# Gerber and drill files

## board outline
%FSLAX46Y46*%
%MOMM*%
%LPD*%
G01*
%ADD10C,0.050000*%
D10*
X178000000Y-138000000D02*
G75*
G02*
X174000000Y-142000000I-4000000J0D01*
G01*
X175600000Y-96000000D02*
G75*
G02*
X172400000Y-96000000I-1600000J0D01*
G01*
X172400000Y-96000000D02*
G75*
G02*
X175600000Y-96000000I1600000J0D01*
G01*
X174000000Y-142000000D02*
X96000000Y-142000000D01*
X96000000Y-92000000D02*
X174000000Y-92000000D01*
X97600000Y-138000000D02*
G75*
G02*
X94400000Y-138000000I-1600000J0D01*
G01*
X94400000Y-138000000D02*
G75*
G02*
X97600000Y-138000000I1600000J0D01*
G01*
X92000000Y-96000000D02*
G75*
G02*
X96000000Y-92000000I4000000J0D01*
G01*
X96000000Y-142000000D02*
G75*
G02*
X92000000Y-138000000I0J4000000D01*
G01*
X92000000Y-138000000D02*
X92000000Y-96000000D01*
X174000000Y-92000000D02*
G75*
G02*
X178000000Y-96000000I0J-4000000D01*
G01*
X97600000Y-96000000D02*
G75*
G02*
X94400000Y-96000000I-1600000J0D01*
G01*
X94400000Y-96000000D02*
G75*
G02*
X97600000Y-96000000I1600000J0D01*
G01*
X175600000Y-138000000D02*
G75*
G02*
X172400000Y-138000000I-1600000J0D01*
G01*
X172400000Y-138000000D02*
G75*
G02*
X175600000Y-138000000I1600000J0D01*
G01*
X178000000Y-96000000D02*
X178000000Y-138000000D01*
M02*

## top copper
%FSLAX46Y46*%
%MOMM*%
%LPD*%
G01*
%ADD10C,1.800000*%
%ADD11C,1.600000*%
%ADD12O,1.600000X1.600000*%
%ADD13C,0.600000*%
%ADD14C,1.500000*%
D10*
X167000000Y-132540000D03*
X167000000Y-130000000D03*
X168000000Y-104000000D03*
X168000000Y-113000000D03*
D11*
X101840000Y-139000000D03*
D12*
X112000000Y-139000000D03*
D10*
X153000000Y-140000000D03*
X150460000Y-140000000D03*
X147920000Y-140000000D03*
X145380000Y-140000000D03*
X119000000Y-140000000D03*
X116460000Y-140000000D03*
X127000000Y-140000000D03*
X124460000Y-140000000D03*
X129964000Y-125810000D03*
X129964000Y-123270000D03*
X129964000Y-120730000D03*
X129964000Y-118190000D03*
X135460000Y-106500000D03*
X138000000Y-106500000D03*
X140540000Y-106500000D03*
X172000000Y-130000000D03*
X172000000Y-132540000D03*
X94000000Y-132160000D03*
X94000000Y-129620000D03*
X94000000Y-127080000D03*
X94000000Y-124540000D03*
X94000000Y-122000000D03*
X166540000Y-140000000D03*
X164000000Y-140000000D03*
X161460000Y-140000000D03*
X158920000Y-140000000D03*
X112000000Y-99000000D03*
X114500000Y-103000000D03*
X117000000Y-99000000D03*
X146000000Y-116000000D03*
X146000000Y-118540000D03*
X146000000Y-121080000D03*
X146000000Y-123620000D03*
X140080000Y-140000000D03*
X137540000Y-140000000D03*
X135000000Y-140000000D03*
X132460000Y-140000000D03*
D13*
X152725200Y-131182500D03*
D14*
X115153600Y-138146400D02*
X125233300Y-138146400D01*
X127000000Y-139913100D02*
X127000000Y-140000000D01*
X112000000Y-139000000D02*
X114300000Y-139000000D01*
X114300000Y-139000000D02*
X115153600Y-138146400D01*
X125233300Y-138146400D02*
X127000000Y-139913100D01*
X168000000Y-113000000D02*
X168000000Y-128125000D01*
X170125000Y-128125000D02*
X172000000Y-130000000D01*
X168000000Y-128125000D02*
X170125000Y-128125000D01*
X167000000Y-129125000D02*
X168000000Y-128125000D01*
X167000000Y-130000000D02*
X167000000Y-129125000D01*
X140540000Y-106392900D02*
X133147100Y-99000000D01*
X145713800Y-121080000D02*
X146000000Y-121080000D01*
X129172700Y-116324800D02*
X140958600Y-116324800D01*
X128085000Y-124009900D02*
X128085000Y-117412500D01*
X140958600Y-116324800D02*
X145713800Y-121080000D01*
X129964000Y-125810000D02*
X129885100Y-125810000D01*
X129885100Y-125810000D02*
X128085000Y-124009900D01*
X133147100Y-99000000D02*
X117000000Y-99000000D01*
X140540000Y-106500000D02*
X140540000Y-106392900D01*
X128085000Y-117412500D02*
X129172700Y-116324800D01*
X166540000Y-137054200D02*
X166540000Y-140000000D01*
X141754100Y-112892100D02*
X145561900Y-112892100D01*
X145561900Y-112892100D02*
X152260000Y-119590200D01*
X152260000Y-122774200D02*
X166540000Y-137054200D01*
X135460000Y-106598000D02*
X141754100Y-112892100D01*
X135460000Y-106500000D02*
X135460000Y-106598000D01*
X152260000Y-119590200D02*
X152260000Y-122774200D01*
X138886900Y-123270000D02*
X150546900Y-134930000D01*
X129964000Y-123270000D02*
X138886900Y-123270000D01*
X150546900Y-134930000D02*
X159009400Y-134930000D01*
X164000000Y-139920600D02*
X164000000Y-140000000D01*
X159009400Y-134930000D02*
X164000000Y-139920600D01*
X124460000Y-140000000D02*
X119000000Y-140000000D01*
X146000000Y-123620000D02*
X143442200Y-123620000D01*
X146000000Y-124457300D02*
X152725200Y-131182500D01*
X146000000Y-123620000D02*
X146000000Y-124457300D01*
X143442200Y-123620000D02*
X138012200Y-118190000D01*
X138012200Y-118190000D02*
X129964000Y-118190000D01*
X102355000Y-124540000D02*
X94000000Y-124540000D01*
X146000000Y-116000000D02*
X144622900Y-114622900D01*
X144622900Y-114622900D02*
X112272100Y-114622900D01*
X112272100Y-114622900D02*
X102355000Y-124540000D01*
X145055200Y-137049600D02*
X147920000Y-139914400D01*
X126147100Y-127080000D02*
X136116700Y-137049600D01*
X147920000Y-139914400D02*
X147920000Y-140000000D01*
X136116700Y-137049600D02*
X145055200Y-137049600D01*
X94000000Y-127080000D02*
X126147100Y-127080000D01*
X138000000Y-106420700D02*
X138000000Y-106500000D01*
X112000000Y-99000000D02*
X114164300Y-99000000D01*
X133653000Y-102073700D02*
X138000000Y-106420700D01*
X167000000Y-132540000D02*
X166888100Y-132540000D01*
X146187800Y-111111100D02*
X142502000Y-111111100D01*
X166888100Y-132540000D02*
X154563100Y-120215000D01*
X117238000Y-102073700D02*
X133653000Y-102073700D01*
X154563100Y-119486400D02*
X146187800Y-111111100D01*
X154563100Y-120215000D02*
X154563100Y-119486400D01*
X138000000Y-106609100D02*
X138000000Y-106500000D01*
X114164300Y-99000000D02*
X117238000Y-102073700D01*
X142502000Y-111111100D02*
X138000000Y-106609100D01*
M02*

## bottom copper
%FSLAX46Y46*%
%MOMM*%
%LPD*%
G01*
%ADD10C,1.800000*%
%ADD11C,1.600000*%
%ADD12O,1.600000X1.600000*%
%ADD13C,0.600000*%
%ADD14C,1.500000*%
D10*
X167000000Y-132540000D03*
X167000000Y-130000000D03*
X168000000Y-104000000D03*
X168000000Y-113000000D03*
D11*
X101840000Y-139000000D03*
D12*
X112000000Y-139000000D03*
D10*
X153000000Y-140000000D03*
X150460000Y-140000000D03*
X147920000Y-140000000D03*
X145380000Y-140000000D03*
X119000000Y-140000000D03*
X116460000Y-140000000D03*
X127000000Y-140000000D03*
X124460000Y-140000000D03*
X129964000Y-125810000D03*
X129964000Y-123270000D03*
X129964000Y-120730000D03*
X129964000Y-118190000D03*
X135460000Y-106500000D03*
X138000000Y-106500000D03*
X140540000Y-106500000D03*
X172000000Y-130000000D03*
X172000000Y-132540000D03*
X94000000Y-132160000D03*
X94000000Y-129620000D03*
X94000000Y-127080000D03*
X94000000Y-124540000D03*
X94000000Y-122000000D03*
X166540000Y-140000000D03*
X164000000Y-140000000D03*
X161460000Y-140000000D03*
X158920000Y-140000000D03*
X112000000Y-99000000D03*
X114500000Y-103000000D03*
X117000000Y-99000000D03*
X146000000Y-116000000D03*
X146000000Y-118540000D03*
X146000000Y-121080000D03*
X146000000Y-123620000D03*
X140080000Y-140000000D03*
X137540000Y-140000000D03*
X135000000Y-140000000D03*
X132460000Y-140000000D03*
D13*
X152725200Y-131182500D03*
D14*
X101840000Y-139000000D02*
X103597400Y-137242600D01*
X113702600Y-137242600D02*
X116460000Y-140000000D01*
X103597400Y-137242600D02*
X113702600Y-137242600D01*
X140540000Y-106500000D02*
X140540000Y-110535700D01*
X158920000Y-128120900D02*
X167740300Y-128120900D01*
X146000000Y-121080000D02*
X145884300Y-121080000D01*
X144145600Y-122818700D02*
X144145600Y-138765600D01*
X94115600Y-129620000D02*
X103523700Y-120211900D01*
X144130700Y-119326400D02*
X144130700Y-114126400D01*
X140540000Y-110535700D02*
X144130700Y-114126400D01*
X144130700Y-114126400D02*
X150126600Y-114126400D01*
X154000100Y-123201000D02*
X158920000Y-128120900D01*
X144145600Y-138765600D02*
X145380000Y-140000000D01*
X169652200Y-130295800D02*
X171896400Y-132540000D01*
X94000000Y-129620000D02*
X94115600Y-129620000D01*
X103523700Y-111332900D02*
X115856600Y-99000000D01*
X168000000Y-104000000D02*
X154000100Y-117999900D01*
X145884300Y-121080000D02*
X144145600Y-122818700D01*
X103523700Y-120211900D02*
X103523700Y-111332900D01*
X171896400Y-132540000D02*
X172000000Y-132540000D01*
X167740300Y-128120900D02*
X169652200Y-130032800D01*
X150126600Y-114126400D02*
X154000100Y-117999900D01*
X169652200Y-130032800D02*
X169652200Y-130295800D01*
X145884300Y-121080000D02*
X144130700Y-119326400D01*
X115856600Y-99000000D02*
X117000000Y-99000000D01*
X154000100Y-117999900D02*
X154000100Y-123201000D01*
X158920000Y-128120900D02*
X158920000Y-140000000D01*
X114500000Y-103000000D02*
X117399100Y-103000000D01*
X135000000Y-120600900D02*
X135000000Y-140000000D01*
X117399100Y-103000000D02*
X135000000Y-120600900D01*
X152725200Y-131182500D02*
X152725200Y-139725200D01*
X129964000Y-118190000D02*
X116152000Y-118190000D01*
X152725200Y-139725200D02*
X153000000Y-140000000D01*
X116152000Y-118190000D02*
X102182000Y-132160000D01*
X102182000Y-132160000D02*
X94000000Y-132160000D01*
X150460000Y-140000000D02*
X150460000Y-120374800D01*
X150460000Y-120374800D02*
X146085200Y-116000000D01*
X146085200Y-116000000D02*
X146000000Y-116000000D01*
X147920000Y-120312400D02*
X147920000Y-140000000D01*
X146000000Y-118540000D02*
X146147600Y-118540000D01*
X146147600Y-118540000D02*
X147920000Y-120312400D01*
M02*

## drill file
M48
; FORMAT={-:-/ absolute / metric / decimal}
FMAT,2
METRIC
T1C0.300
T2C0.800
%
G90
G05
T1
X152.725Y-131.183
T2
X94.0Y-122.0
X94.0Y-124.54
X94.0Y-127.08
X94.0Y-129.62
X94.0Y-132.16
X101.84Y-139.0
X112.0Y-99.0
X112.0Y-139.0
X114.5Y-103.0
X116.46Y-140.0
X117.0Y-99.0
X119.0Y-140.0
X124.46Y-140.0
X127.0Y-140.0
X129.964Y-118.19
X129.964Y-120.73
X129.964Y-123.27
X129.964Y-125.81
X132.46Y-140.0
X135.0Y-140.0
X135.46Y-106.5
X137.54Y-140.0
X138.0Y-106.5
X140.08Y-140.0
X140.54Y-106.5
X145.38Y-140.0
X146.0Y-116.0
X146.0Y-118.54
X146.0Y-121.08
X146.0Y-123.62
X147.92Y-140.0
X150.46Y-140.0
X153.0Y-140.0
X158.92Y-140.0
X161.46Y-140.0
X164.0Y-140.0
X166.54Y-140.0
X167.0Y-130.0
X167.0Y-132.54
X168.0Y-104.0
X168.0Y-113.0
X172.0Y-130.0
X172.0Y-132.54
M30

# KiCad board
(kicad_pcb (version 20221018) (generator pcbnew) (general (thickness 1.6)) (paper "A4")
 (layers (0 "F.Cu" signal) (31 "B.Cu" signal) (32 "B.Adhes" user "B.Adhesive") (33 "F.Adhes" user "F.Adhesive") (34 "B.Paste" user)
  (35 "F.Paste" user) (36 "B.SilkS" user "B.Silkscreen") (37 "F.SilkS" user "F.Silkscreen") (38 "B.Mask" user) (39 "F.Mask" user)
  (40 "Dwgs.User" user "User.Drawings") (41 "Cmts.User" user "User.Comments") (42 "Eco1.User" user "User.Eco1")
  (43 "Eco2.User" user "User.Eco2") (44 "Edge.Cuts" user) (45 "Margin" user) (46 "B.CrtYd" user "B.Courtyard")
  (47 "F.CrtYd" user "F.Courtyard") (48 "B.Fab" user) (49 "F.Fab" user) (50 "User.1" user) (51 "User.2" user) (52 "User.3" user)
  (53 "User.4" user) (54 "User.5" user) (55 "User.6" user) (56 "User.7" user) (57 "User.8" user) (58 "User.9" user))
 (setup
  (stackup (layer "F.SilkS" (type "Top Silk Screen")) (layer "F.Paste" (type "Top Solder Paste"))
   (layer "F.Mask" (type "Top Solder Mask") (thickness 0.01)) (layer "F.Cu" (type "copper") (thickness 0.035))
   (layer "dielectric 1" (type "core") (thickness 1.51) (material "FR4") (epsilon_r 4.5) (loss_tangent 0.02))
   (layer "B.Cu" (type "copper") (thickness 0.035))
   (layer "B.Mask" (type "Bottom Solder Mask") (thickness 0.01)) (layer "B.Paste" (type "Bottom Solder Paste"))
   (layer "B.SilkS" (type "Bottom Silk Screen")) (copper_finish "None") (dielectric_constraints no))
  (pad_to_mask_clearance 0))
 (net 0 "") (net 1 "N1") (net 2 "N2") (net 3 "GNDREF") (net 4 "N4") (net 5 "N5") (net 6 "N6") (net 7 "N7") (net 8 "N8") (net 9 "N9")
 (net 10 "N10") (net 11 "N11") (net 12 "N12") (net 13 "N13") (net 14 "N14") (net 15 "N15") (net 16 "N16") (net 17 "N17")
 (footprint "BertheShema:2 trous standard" (layer "F.Cu") (at 167 132.54)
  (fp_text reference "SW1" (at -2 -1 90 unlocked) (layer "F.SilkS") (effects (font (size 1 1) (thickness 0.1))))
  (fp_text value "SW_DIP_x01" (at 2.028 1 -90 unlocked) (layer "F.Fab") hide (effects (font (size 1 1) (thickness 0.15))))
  (pad "1" thru_hole circle (at 0 0) (size 1.8 1.8) (drill 0.8) (layers "*.Cu" "*.Mask") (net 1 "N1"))
  (pad "2" thru_hole circle (at 0 -2.54) (size 1.8 1.8) (drill 0.8) (layers "*.Cu" "*.Mask") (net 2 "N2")))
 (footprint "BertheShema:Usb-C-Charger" (layer "F.Cu") (at 175 107 -90)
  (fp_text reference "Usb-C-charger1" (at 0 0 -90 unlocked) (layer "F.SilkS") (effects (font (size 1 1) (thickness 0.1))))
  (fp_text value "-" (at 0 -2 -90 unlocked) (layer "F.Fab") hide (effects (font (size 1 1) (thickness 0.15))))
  (pad "1" thru_hole circle (at -3 7 270) (size 1.8 1.8) (drill 0.8) (layers "*.Cu" "*.Mask") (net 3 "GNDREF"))
  (pad "2" thru_hole circle (at 6 7 270) (size 1.8 1.8) (drill 0.8) (layers "*.Cu" "*.Mask") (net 2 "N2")))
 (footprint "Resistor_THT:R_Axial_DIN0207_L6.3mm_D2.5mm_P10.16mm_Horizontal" (layer "F.Cu") (at 101.84 139)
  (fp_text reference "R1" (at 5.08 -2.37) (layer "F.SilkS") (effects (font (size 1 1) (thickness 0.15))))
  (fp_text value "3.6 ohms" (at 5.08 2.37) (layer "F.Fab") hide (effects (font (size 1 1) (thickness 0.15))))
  (pad "1" thru_hole circle (at 0 0) (size 1.6 1.6) (drill 0.8) (layers "*.Cu" "*.Mask") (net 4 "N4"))
  (pad "2" thru_hole oval (at 10.16 0) (size 1.6 1.6) (drill 0.8) (layers "*.Cu" "*.Mask") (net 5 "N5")))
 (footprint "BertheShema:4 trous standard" (layer "F.Cu") (at 150.46 140 90)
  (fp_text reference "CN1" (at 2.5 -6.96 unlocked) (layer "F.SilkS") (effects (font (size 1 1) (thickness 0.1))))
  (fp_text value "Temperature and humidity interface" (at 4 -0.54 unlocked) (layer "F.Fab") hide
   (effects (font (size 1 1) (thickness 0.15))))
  (pad "1" thru_hole circle (at 0 2.54 90) (size 1.8 1.8) (drill 0.8) (layers "*.Cu" "*.Mask") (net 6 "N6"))
  (pad "2" thru_hole circle (at 0 0 90) (size 1.8 1.8) (drill 0.8) (layers "*.Cu" "*.Mask") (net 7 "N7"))
  (pad "3" thru_hole circle (at 0 -2.54 90) (size 1.8 1.8) (drill 0.8) (layers "*.Cu" "*.Mask") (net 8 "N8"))
  (pad "4" thru_hole circle (at 0 -5.08 90) (size 1.8 1.8) (drill 0.8) (layers "*.Cu" "*.Mask") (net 3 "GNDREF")))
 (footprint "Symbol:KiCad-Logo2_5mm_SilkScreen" (layer "F.Cu") (at 154 106)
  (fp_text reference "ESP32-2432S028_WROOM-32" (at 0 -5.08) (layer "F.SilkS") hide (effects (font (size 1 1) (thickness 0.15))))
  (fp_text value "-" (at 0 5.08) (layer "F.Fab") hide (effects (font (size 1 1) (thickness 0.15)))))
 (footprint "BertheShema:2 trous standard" (layer "F.Cu") (at 119 140 90)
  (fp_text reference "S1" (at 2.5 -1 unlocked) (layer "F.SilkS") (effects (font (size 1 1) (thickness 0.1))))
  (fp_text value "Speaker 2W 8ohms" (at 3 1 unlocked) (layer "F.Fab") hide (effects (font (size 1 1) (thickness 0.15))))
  (pad "1" thru_hole circle (at 0 0 90) (size 1.8 1.8) (drill 0.8) (layers "*.Cu" "*.Mask") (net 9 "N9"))
  (pad "2" thru_hole circle (at 0 -2.54 90) (size 1.8 1.8) (drill 0.8) (layers "*.Cu" "*.Mask") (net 4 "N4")))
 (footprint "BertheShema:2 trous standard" (layer "F.Cu") (at 127 140 90)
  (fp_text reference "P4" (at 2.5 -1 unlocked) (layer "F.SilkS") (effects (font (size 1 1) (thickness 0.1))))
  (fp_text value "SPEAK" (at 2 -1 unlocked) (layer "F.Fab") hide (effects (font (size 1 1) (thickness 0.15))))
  (pad "1" thru_hole circle (at 0 0 90) (size 1.8 1.8) (drill 0.8) (layers "*.Cu" "*.Mask") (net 5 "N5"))
  (pad "2" thru_hole circle (at 0 -2.54 90) (size 1.8 1.8) (drill 0.8) (layers "*.Cu" "*.Mask") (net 9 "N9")))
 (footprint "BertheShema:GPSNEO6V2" (layer "F.Cu") (at 128.44 122 90)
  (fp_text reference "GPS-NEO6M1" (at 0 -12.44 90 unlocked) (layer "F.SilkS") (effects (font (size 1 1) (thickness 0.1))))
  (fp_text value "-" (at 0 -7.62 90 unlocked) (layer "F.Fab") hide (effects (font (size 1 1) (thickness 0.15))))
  (pad "1" thru_hole circle (at -3.81 1.524 90) (size 1.8 1.8) (drill 0.8) (layers "*.Cu" "*.Mask") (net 3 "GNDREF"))
  (pad "2" thru_hole circle (at -1.27 1.524 90) (size 1.8 1.8) (drill 0.8) (layers "*.Cu" "*.Mask") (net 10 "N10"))
  (pad "3" thru_hole circle (at 1.27 1.524 90) (size 1.8 1.8) (drill 0.8) (layers "*.Cu" "*.Mask") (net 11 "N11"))
  (pad "4" thru_hole circle (at 3.81 1.524 90) (size 1.8 1.8) (drill 0.8) (layers "*.Cu" "*.Mask") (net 6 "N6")))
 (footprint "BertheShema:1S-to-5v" (layer "F.Cu") (at 138 102.5)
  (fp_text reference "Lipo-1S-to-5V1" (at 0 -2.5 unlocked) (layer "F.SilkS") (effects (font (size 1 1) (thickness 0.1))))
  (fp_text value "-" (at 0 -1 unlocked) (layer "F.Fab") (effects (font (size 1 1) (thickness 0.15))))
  (pad "1" thru_hole circle (at -2.54 4) (size 1.8 1.8) (drill 0.8) (layers "*.Cu" "*.Mask") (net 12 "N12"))
  (pad "2" thru_hole circle (at 0 4) (size 1.8 1.8) (drill 0.8) (layers "*.Cu" "*.Mask") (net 1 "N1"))
  (pad "3" thru_hole circle (at 2.54 4) (size 1.8 1.8) (drill 0.8) (layers "*.Cu" "*.Mask") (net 3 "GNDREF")))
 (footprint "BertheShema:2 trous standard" (layer "F.Cu") (at 172 130 180)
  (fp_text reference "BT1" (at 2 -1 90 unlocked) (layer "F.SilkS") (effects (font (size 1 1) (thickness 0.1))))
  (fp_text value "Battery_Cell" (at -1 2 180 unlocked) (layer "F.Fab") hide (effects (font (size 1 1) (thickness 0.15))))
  (pad "1" thru_hole circle (at 0 0 180) (size 1.8 1.8) (drill 0.8) (layers "*.Cu" "*.Mask") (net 2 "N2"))
  (pad "2" thru_hole circle (at 0 -2.54 180) (size 1.8 1.8) (drill 0.8) (layers "*.Cu" "*.Mask") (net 3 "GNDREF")))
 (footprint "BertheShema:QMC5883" (layer "F.Cu") (at 88.92 127.08 90)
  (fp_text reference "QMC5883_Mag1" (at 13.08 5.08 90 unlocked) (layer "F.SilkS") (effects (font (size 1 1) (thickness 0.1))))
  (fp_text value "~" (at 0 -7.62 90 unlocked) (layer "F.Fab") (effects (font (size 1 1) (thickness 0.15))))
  (pad "1" thru_hole circle (at -5.08 5.08 90) (size 1.8 1.8) (drill 0.8) (layers "*.Cu" "*.Mask") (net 6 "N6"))
  (pad "2" thru_hole circle (at -2.54 5.08 90) (size 1.8 1.8) (drill 0.8) (layers "*.Cu" "*.Mask") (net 3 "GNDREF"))
  (pad "3" thru_hole circle (at 0 5.08 90) (size 1.8 1.8) (drill 0.8) (layers "*.Cu" "*.Mask") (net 8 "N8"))
  (pad "4" thru_hole circle (at 2.54 5.08 90) (size 1.8 1.8) (drill 0.8) (layers "*.Cu" "*.Mask") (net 7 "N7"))
  (pad "5" thru_hole circle (at 5.08 5.08 90) (size 1.8 1.8) (drill 0.8) (layers "*.Cu" "*.Mask")))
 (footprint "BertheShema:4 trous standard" (layer "F.Cu") (at 164 140 90)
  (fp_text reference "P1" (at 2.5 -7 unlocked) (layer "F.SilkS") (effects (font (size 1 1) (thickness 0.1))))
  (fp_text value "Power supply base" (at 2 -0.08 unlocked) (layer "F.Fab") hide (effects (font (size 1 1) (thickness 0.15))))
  (pad "1" thru_hole circle (at 0 2.54 90) (size 1.8 1.8) (drill 0.8) (layers "*.Cu" "*.Mask") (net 12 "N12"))
  (pad "2" thru_hole circle (at 0 0 90) (size 1.8 1.8) (drill 0.8) (layers "*.Cu" "*.Mask") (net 10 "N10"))
  (pad "3" thru_hole circle (at 0 -2.54 90) (size 1.8 1.8) (drill 0.8) (layers "*.Cu" "*.Mask") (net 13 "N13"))
  (pad "4" thru_hole circle (at 0 -5.08 90) (size 1.8 1.8) (drill 0.8) (layers "*.Cu" "*.Mask") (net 3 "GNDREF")))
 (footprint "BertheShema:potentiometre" (layer "F.Cu") (at 114.5 99.5)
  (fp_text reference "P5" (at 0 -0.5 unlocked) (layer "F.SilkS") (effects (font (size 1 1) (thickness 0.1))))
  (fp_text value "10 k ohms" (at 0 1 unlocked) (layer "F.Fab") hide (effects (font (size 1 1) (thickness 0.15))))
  (pad "1" thru_hole circle (at -2.5 -0.5) (size 1.8 1.8) (drill 0.8) (layers "*.Cu" "*.Mask") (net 1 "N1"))
  (pad "2" thru_hole circle (at 0 3.5) (size 1.8 1.8) (drill 0.8) (layers "*.Cu" "*.Mask") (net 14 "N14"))
  (pad "3" thru_hole circle (at 2.5 -0.5) (size 1.8 1.8) (drill 0.8) (layers "*.Cu" "*.Mask") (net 3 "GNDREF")))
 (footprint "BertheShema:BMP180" (layer "F.Cu") (at 147.524 119.81 -90)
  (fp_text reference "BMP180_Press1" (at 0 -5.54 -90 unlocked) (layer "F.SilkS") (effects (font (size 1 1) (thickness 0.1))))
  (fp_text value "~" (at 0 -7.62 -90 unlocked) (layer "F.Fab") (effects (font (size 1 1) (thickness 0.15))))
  (pad "1" thru_hole circle (at -3.81 1.524 270) (size 1.8 1.8) (drill 0.8) (layers "*.Cu" "*.Mask") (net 7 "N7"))
  (pad "2" thru_hole circle (at -1.27 1.524 270) (size 1.8 1.8) (drill 0.8) (layers "*.Cu" "*.Mask") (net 8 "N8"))
  (pad "3" thru_hole circle (at 1.27 1.524 270) (size 1.8 1.8) (drill 0.8) (layers "*.Cu" "*.Mask") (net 3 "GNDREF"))
  (pad "4" thru_hole circle (at 3.81 1.524 270) (size 1.8 1.8) (drill 0.8) (layers "*.Cu" "*.Mask") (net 6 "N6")))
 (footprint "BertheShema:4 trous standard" (layer "F.Cu") (at 137.54 140 90)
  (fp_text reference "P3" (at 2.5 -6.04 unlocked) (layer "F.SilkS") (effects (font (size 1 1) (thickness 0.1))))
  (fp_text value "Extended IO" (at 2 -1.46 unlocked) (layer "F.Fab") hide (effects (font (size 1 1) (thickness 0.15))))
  (pad "1" thru_hole circle (at 0 2.54 90) (size 1.8 1.8) (drill 0.8) (layers "*.Cu" "*.Mask") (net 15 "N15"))
  (pad "2" thru_hole circle (at 0 0 90) (size 1.8 1.8) (drill 0.8) (layers "*.Cu" "*.Mask") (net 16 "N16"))
  (pad "3" thru_hole circle (at 0 -2.54 90) (size 1.8 1.8) (drill 0.8) (layers "*.Cu" "*.Mask") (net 14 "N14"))
  (pad "4" thru_hole circle (at 0 -5.08 90) (size 1.8 1.8) (drill 0.8) (layers "*.Cu" "*.Mask") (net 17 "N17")))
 (gr_arc (start 178 138) (mid 176.828427 140.828427) (end 174 142) (stroke (width 0.05) (type default)) (layer "Edge.Cuts"))
 (gr_circle (center 174 96) (end 175.6 96) (stroke (width 0.05) (type default)) (fill none) (layer "Edge.Cuts"))
 (gr_line (start 174 142) (end 96 142) (stroke (width 0.05) (type default)) (layer "Edge.Cuts"))
 (gr_line (start 96 92) (end 174 92) (stroke (width 0.05) (type default)) (layer "Edge.Cuts"))
 (gr_circle (center 96 138) (end 97.6 138) (stroke (width 0.05) (type default)) (fill none) (layer "Edge.Cuts"))
 (gr_arc (start 92 96) (mid 93.171573 93.171573) (end 96 92) (stroke (width 0.05) (type default)) (layer "Edge.Cuts"))
 (gr_arc (start 96 142) (mid 93.171573 140.828427) (end 92 138) (stroke (width 0.05) (type default)) (layer "Edge.Cuts"))
 (gr_line (start 92 138) (end 92 96) (stroke (width 0.05) (type default)) (layer "Edge.Cuts"))
 (gr_arc (start 174 92) (mid 176.828427 93.171573) (end 178 96) (stroke (width 0.05) (type default)) (layer "Edge.Cuts"))
 (gr_circle (center 96 96) (end 97.6 96) (stroke (width 0.05) (type default)) (fill none) (layer "Edge.Cuts"))
 (gr_circle (center 174 138) (end 175.6 138) (stroke (width 0.05) (type default)) (fill none) (layer "Edge.Cuts"))
 (gr_line (start 178 96) (end 178 138) (stroke (width 0.05) (type default)) (layer "Edge.Cuts"))
 (segment (start 101.84 139) (end 103.5974 137.2426) (width 1.5) (layer "B.Cu") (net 4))
 (segment (start 113.7026 137.2426) (end 116.46 140) (width 1.5) (layer "B.Cu") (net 4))
 (segment (start 103.5974 137.2426) (end 113.7026 137.2426) (width 1.5) (layer "B.Cu") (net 4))
 (segment (start 115.1536 138.1464) (end 125.2333 138.1464) (width 1.5) (layer "F.Cu") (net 5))
 (segment (start 127 139.9131) (end 127 140) (width 1.5) (layer "F.Cu") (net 5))
 (segment (start 112 139) (end 114.3 139) (width 1.5) (layer "F.Cu") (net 5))
 (segment (start 114.3 139) (end 115.1536 138.1464) (width 1.5) (layer "F.Cu") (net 5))
 (segment (start 125.2333 138.1464) (end 127 139.9131) (width 1.5) (layer "F.Cu") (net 5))
 (segment (start 168 113) (end 168 128.125) (width 1.5) (layer "F.Cu") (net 2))
 (segment (start 170.125 128.125) (end 172 130) (width 1.5) (layer "F.Cu") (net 2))
 (segment (start 168 128.125) (end 170.125 128.125) (width 1.5) (layer "F.Cu") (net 2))
 (segment (start 167 129.125) (end 168 128.125) (width 1.5) (layer "F.Cu") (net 2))
 (segment (start 167 130) (end 167 129.125) (width 1.5) (layer "F.Cu") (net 2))
 (segment (start 140.54 106.3929) (end 133.1471 99) (width 1.5) (layer "F.Cu") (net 3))
 (segment (start 145.7138 121.08) (end 146 121.08) (width 1.5) (layer "F.Cu") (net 3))
 (segment (start 129.1727 116.3248) (end 140.9586 116.3248) (width 1.5) (layer "F.Cu") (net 3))
 (segment (start 128.085 124.0099) (end 128.085 117.4125) (width 1.5) (layer "F.Cu") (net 3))
 (segment (start 140.9586 116.3248) (end 145.7138 121.08) (width 1.5) (layer "F.Cu") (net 3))
 (segment (start 129.964 125.81) (end 129.8851 125.81) (width 1.5) (layer "F.Cu") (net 3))
 (segment (start 129.8851 125.81) (end 128.085 124.0099) (width 1.5) (layer "F.Cu") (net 3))
 (segment (start 133.1471 99) (end 117 99) (width 1.5) (layer "F.Cu") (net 3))
 (segment (start 140.54 106.5) (end 140.54 106.3929) (width 1.5) (layer "F.Cu") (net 3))
 (segment (start 128.085 117.4125) (end 129.1727 116.3248) (width 1.5) (layer "F.Cu") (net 3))
 (segment (start 140.54 106.5) (end 140.54 110.5357) (width 1.5) (layer "B.Cu") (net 3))
 (segment (start 158.92 128.1209) (end 167.7403 128.1209) (width 1.5) (layer "B.Cu") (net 3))
 (segment (start 146 121.08) (end 145.8843 121.08) (width 1.5) (layer "B.Cu") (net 3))
 (segment (start 144.1456 122.8187) (end 144.1456 138.7656) (width 1.5) (layer "B.Cu") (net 3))
 (segment (start 94.1156 129.62) (end 103.5237 120.2119) (width 1.5) (layer "B.Cu") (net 3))
 (segment (start 144.1307 119.3264) (end 144.1307 114.1264) (width 1.5) (layer "B.Cu") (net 3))
 (segment (start 140.54 110.5357) (end 144.1307 114.1264) (width 1.5) (layer "B.Cu") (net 3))
 (segment (start 144.1307 114.1264) (end 150.1266 114.1264) (width 1.5) (layer "B.Cu") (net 3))
 (segment (start 154.0001 123.201) (end 158.92 128.1209) (width 1.5) (layer "B.Cu") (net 3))
 (segment (start 144.1456 138.7656) (end 145.38 140) (width 1.5) (layer "B.Cu") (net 3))
 (segment (start 169.6522 130.2958) (end 171.8964 132.54) (width 1.5) (layer "B.Cu") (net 3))
 (segment (start 94 129.62) (end 94.1156 129.62) (width 1.5) (layer "B.Cu") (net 3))
 (segment (start 103.5237 111.3329) (end 115.8566 99) (width 1.5) (layer "B.Cu") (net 3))
 (segment (start 168 104) (end 154.0001 117.9999) (width 1.5) (layer "B.Cu") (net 3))
 (segment (start 145.8843 121.08) (end 144.1456 122.8187) (width 1.5) (layer "B.Cu") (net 3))
 (segment (start 103.5237 120.2119) (end 103.5237 111.3329) (width 1.5) (layer "B.Cu") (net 3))
 (segment (start 171.8964 132.54) (end 172 132.54) (width 1.5) (layer "B.Cu") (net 3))
 (segment (start 167.7403 128.1209) (end 169.6522 130.0328) (width 1.5) (layer "B.Cu") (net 3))
 (segment (start 150.1266 114.1264) (end 154.0001 117.9999) (width 1.5) (layer "B.Cu") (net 3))
 (segment (start 169.6522 130.0328) (end 169.6522 130.2958) (width 1.5) (layer "B.Cu") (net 3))
 (segment (start 145.8843 121.08) (end 144.1307 119.3264) (width 1.5) (layer "B.Cu") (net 3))
 (segment (start 115.8566 99) (end 117 99) (width 1.5) (layer "B.Cu") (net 3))
 (segment (start 154.0001 117.9999) (end 154.0001 123.201) (width 1.5) (layer "B.Cu") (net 3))
 (segment (start 158.92 128.1209) (end 158.92 140) (width 1.5) (layer "B.Cu") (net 3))
 (segment (start 166.54 137.0542) (end 166.54 140) (width 1.5) (layer "F.Cu") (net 12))
 (segment (start 141.7541 112.8921) (end 145.5619 112.8921) (width 1.5) (layer "F.Cu") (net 12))
 (segment (start 145.5619 112.8921) (end 152.26 119.5902) (width 1.5) (layer "F.Cu") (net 12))
 (segment (start 152.26 122.7742) (end 166.54 137.0542) (width 1.5) (layer "F.Cu") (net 12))
 (segment (start 135.46 106.598) (end 141.7541 112.8921) (width 1.5) (layer "F.Cu") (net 12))
 (segment (start 135.46 106.5) (end 135.46 106.598) (width 1.5) (layer "F.Cu") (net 12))
 (segment (start 152.26 119.5902) (end 152.26 122.7742) (width 1.5) (layer "F.Cu") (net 12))
 (segment (start 138.8869 123.27) (end 150.5469 134.93) (width 1.5) (layer "F.Cu") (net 10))
 (segment (start 129.964 123.27) (end 138.8869 123.27) (width 1.5) (layer "F.Cu") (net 10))
 (segment (start 150.5469 134.93) (end 159.0094 134.93) (width 1.5) (layer "F.Cu") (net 10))
 (segment (start 164 139.9206) (end 164 140) (width 1.5) (layer "F.Cu") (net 10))
 (segment (start 159.0094 134.93) (end 164 139.9206) (width 1.5) (layer "F.Cu") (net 10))
 (segment (start 114.5 103) (end 117.3991 103) (width 1.5) (layer "B.Cu") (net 14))
 (segment (start 135 120.6009) (end 135 140) (width 1.5) (layer "B.Cu") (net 14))
 (segment (start 117.3991 103) (end 135 120.6009) (width 1.5) (layer "B.Cu") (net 14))
 (segment (start 124.46 140) (end 119 140) (width 1.5) (layer "F.Cu") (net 9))
 (segment (start 146 123.62) (end 143.4422 123.62) (width 1.5) (layer "F.Cu") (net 6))
 (segment (start 146 124.4573) (end 152.7252 131.1825) (width 1.5) (layer "F.Cu") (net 6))
 (segment (start 146 123.62) (end 146 124.4573) (width 1.5) (layer "F.Cu") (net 6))
 (segment (start 143.4422 123.62) (end 138.0122 118.19) (width 1.5) (layer "F.Cu") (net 6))
 (segment (start 138.0122 118.19) (end 129.964 118.19) (width 1.5) (layer "F.Cu") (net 6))
 (via (at 152.7252 131.1825) (size 0.6) (drill 0.3) (layers "F.Cu" "B.Cu") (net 6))
 (segment (start 152.7252 131.1825) (end 152.7252 139.7252) (width 1.5) (layer "B.Cu") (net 6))
 (segment (start 129.964 118.19) (end 116.152 118.19) (width 1.5) (layer "B.Cu") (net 6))
 (segment (start 152.7252 139.7252) (end 153 140) (width 1.5) (layer "B.Cu") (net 6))
 (segment (start 116.152 118.19) (end 102.182 132.16) (width 1.5) (layer "B.Cu") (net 6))
 (segment (start 102.182 132.16) (end 94 132.16) (width 1.5) (layer "B.Cu") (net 6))
 (segment (start 102.355 124.54) (end 94 124.54) (width 1.5) (layer "F.Cu") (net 7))
 (segment (start 146 116) (end 144.6229 114.6229) (width 1.5) (layer "F.Cu") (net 7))
 (segment (start 144.6229 114.6229) (end 112.2721 114.6229) (width 1.5) (layer "F.Cu") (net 7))
 (segment (start 112.2721 114.6229) (end 102.355 124.54) (width 1.5) (layer "F.Cu") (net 7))
 (segment (start 150.46 140) (end 150.46 120.3748) (width 1.5) (layer "B.Cu") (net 7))
 (segment (start 150.46 120.3748) (end 146.0852 116) (width 1.5) (layer "B.Cu") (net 7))
 (segment (start 146.0852 116) (end 146 116) (width 1.5) (layer "B.Cu") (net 7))
 (segment (start 145.0552 137.0496) (end 147.92 139.9144) (width 1.5) (layer "F.Cu") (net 8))
 (segment (start 126.1471 127.08) (end 136.1167 137.0496) (width 1.5) (layer "F.Cu") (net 8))
 (segment (start 147.92 139.9144) (end 147.92 140) (width 1.5) (layer "F.Cu") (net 8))
 (segment (start 136.1167 137.0496) (end 145.0552 137.0496) (width 1.5) (layer "F.Cu") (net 8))
 (segment (start 94 127.08) (end 126.1471 127.08) (width 1.5) (layer "F.Cu") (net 8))
 (segment (start 147.92 120.3124) (end 147.92 140) (width 1.5) (layer "B.Cu") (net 8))
 (segment (start 146 118.54) (end 146.1476 118.54) (width 1.5) (layer "B.Cu") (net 8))
 (segment (start 146.1476 118.54) (end 147.92 120.3124) (width 1.5) (layer "B.Cu") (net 8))
 (segment (start 138 106.4207) (end 138 106.5) (width 1.5) (layer "F.Cu") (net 1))
 (segment (start 112 99) (end 114.1643 99) (width 1.5) (layer "F.Cu") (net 1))
 (segment (start 133.653 102.0737) (end 138 106.4207) (width 1.5) (layer "F.Cu") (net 1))
 (segment (start 167 132.54) (end 166.8881 132.54) (width 1.5) (layer "F.Cu") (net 1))
 (segment (start 146.1878 111.1111) (end 142.502 111.1111) (width 1.5) (layer "F.Cu") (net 1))
 (segment (start 166.8881 132.54) (end 154.5631 120.215) (width 1.5) (layer "F.Cu") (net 1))
 (segment (start 117.238 102.0737) (end 133.653 102.0737) (width 1.5) (layer "F.Cu") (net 1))
 (segment (start 154.5631 119.4864) (end 146.1878 111.1111) (width 1.5) (layer "F.Cu") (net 1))
 (segment (start 154.5631 120.215) (end 154.5631 119.4864) (width 1.5) (layer "F.Cu") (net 1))
 (segment (start 138 106.6091) (end 138 106.5) (width 1.5) (layer "F.Cu") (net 1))
 (segment (start 114.1643 99) (end 117.238 102.0737) (width 1.5) (layer "F.Cu") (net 1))
 (segment (start 142.502 111.1111) (end 138 106.6091) (width 1.5) (layer "F.Cu") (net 1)))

